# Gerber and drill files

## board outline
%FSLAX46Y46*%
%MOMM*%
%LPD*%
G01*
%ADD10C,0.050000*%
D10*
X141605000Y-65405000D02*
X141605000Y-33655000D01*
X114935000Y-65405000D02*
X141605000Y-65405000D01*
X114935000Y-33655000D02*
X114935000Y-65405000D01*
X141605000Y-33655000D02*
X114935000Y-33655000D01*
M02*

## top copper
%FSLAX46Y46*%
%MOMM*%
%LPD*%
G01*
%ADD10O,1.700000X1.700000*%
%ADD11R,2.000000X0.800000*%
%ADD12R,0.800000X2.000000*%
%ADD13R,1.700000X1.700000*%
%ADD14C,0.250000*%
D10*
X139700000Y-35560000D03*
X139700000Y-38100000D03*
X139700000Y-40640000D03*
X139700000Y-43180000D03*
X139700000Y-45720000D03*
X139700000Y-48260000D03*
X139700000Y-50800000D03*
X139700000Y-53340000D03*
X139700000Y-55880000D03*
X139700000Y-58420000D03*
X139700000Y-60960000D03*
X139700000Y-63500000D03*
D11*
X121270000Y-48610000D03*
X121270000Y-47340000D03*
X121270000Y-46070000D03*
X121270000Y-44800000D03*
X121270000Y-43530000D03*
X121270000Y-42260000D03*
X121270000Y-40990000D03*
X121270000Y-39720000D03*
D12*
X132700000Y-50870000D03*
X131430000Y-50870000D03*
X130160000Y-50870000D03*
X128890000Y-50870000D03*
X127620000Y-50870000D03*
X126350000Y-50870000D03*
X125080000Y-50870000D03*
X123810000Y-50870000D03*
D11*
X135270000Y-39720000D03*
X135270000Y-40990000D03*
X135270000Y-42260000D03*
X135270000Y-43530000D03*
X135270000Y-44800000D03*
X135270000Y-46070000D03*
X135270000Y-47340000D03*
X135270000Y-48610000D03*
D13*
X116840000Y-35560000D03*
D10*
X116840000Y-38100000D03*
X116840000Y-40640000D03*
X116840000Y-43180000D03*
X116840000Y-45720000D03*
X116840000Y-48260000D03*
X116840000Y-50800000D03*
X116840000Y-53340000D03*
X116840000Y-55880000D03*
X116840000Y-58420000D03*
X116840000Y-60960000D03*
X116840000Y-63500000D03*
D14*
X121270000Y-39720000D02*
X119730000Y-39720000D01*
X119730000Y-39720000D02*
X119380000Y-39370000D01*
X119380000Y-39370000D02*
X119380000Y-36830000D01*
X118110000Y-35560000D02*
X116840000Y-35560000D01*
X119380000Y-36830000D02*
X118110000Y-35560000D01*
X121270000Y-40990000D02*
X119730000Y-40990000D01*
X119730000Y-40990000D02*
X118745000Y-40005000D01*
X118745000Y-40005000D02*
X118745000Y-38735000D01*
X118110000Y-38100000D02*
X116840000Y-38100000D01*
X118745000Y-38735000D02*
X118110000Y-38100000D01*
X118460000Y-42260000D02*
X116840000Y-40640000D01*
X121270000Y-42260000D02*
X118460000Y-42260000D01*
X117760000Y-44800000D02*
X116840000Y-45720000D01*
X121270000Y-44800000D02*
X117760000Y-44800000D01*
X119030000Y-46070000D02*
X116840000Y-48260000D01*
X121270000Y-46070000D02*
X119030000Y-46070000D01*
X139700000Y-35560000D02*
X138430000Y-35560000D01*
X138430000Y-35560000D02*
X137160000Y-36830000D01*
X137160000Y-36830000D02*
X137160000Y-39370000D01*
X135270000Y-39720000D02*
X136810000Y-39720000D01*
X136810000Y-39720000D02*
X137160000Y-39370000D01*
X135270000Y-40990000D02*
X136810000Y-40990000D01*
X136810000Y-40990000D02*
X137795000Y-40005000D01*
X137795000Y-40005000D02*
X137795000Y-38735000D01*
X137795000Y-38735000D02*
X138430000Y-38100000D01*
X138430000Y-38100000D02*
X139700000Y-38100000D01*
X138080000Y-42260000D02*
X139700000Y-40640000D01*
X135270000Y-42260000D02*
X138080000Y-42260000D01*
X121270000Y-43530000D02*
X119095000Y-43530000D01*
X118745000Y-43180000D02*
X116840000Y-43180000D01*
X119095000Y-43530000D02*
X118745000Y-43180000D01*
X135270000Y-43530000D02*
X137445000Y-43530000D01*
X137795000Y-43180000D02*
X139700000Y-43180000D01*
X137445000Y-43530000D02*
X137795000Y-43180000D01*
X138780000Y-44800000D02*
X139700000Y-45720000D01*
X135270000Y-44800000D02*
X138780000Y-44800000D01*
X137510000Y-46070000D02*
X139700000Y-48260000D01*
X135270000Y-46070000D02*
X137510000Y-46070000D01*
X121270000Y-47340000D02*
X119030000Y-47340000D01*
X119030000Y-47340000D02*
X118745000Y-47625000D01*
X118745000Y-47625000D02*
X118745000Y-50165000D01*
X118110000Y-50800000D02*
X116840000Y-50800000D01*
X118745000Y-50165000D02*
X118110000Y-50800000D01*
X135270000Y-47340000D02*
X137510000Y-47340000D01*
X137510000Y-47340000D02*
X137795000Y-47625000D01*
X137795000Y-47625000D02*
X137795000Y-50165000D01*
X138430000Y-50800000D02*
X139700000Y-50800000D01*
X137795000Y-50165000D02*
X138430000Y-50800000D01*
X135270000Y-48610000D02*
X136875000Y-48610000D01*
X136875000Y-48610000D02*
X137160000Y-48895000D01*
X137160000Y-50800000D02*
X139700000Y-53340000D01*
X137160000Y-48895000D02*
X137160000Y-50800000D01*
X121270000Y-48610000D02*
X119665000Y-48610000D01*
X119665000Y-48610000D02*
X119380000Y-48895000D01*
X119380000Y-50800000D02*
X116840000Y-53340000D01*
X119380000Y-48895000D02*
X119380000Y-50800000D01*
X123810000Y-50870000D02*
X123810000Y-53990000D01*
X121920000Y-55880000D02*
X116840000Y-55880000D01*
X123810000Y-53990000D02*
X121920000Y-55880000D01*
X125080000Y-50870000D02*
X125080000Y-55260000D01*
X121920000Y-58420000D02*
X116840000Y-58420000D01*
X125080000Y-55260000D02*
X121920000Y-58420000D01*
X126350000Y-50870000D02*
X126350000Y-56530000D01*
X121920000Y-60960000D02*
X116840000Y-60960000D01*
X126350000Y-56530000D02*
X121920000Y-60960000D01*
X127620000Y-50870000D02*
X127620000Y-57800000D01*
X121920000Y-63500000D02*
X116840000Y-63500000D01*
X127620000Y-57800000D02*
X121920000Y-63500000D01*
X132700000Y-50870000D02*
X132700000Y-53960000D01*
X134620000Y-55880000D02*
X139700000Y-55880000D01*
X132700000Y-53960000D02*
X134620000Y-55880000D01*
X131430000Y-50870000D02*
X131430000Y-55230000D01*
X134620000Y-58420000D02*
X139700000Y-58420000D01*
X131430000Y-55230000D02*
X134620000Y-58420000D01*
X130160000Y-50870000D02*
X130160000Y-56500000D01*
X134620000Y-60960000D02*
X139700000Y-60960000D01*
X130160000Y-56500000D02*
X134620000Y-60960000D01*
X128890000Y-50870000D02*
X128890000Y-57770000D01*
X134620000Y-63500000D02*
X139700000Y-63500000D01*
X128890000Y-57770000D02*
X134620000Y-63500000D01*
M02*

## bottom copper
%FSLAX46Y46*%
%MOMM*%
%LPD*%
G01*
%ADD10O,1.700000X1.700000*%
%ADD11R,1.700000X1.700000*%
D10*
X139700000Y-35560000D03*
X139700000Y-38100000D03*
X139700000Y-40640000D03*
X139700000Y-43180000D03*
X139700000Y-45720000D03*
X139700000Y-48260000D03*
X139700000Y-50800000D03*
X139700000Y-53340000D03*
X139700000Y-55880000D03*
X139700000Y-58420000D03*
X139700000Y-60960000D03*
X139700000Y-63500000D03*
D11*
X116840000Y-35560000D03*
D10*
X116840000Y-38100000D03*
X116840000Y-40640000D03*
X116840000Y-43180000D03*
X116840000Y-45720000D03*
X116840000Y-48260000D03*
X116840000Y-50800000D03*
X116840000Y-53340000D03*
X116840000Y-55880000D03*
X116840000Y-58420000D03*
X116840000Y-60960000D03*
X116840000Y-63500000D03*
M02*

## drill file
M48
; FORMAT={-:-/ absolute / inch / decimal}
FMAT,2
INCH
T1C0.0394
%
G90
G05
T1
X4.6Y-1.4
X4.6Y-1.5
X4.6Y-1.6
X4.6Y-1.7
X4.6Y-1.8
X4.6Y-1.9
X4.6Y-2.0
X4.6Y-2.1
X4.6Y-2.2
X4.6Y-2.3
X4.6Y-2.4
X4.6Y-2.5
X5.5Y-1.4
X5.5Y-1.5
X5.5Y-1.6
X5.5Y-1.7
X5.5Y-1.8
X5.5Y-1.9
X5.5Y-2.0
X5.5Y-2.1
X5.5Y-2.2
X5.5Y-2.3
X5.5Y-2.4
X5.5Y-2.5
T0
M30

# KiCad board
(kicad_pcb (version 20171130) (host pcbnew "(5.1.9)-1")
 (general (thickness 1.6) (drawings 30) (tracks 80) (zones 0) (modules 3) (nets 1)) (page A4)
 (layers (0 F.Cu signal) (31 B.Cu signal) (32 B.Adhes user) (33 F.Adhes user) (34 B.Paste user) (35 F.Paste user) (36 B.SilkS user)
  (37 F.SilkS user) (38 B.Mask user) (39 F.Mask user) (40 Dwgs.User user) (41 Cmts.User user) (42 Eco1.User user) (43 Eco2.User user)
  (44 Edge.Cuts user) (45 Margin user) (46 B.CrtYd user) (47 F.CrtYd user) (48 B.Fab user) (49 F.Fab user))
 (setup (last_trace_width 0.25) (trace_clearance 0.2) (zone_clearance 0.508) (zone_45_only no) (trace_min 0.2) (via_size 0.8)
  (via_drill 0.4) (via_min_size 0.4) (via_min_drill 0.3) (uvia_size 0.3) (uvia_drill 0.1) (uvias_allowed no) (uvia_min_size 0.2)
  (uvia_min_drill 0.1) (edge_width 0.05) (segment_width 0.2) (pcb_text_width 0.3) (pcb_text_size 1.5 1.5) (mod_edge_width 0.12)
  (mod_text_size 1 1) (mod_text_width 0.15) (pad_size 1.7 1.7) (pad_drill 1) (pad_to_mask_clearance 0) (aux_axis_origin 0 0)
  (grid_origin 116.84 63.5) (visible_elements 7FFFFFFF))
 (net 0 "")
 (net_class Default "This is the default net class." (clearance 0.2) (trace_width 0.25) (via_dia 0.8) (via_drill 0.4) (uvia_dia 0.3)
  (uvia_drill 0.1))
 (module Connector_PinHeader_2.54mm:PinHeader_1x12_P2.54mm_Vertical (layer B.Cu) (at 139.7 63.5)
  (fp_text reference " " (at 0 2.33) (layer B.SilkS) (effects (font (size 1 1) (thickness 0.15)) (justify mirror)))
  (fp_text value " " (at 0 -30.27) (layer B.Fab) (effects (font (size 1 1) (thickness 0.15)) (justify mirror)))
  (pad 12 thru_hole oval (at 0 -27.94) (size 1.7 1.7) (drill 1) (layers *.Cu *.Mask))
  (pad 11 thru_hole oval (at 0 -25.4) (size 1.7 1.7) (drill 1) (layers *.Cu *.Mask))
  (pad 10 thru_hole oval (at 0 -22.86) (size 1.7 1.7) (drill 1) (layers *.Cu *.Mask))
  (pad 9 thru_hole oval (at 0 -20.32) (size 1.7 1.7) (drill 1) (layers *.Cu *.Mask))
  (pad 8 thru_hole oval (at 0 -17.78) (size 1.7 1.7) (drill 1) (layers *.Cu *.Mask))
  (pad 7 thru_hole oval (at 0 -15.24) (size 1.7 1.7) (drill 1) (layers *.Cu *.Mask))
  (pad 6 thru_hole oval (at 0 -12.7) (size 1.7 1.7) (drill 1) (layers *.Cu *.Mask))
  (pad 5 thru_hole oval (at 0 -10.16) (size 1.7 1.7) (drill 1) (layers *.Cu *.Mask))
  (pad 4 thru_hole oval (at 0 -7.62) (size 1.7 1.7) (drill 1) (layers *.Cu *.Mask))
  (pad 3 thru_hole oval (at 0 -5.08) (size 1.7 1.7) (drill 1) (layers *.Cu *.Mask))
  (pad 2 thru_hole oval (at 0 -2.54) (size 1.7 1.7) (drill 1) (layers *.Cu *.Mask))
  (pad 1 thru_hole oval (at 0 0) (size 1.7 1.7) (drill 1) (layers *.Cu *.Mask)))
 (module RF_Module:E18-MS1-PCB (layer F.Cu) (at 128.27 39.37)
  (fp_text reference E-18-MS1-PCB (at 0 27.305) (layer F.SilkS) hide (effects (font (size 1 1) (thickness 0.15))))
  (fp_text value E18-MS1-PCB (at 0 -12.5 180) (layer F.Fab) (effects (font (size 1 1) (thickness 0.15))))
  (pad 8 smd rect (at -7 9.24 270) (size 0.8 2) (layers F.Cu F.Paste F.Mask))
  (pad 7 smd rect (at -7 7.97 270) (size 0.8 2) (layers F.Cu F.Paste F.Mask))
  (pad 6 smd rect (at -7 6.7 270) (size 0.8 2) (layers F.Cu F.Paste F.Mask))
  (pad 5 smd rect (at -7 5.43 270) (size 0.8 2) (layers F.Cu F.Paste F.Mask))
  (pad 4 smd rect (at -7 4.16 270) (size 0.8 2) (layers F.Cu F.Paste F.Mask))
  (pad 3 smd rect (at -7 2.89 270) (size 0.8 2) (layers F.Cu F.Paste F.Mask))
  (pad 2 smd rect (at -7 1.62 270) (size 0.8 2) (layers F.Cu F.Paste F.Mask))
  (pad 1 smd rect (at -7 0.35 270) (size 0.8 2) (layers F.Cu F.Paste F.Mask))
  (pad 16 smd rect (at 4.43 11.5 180) (size 0.8 2) (layers F.Cu F.Paste F.Mask))
  (pad 15 smd rect (at 3.16 11.5 180) (size 0.8 2) (layers F.Cu F.Paste F.Mask))
  (pad 14 smd rect (at 1.89 11.5 180) (size 0.8 2) (layers F.Cu F.Paste F.Mask))
  (pad 13 smd rect (at 0.62 11.5 180) (size 0.8 2) (layers F.Cu F.Paste F.Mask))
  (pad 12 smd rect (at -0.65 11.5 180) (size 0.8 2) (layers F.Cu F.Paste F.Mask))
  (pad 11 smd rect (at -1.92 11.5 180) (size 0.8 2) (layers F.Cu F.Paste F.Mask))
  (pad 10 smd rect (at -3.19 11.5 180) (size 0.8 2) (layers F.Cu F.Paste F.Mask))
  (pad 9 smd rect (at -4.46 11.5 180) (size 0.8 2) (layers F.Cu F.Paste F.Mask))
  (pad 24 smd rect (at 7 0.35 90) (size 0.8 2) (layers F.Cu F.Paste F.Mask))
  (pad 23 smd rect (at 7 1.62 90) (size 0.8 2) (layers F.Cu F.Paste F.Mask))
  (pad 22 smd rect (at 7 2.89 90) (size 0.8 2) (layers F.Cu F.Paste F.Mask))
  (pad 21 smd rect (at 7 4.16 90) (size 0.8 2) (layers F.Cu F.Paste F.Mask))
  (pad 20 smd rect (at 7 5.43 90) (size 0.8 2) (layers F.Cu F.Paste F.Mask))
  (pad 19 smd rect (at 7 6.7 90) (size 0.8 2) (layers F.Cu F.Paste F.Mask))
  (pad 18 smd rect (at 7 7.97 90) (size 0.8 2) (layers F.Cu F.Paste F.Mask))
  (pad 17 smd rect (at 7 9.24 90) (size 0.8 2) (layers F.Cu F.Paste F.Mask)))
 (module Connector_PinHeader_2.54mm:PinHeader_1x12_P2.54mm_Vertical (layer B.Cu) (at 116.84 63.5)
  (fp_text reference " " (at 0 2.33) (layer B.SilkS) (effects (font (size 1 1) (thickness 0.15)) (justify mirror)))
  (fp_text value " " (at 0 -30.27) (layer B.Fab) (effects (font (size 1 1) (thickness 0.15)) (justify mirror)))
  (pad 12 thru_hole rect (at 0 -27.94) (size 1.7 1.7) (drill 1) (layers *.Cu *.Mask))
  (pad 11 thru_hole oval (at 0 -25.4) (size 1.7 1.7) (drill 1) (layers *.Cu *.Mask))
  (pad 10 thru_hole oval (at 0 -22.86) (size 1.7 1.7) (drill 1) (layers *.Cu *.Mask))
  (pad 9 thru_hole oval (at 0 -20.32) (size 1.7 1.7) (drill 1) (layers *.Cu *.Mask))
  (pad 8 thru_hole oval (at 0 -17.78) (size 1.7 1.7) (drill 1) (layers *.Cu *.Mask))
  (pad 7 thru_hole oval (at 0 -15.24) (size 1.7 1.7) (drill 1) (layers *.Cu *.Mask))
  (pad 6 thru_hole oval (at 0 -12.7) (size 1.7 1.7) (drill 1) (layers *.Cu *.Mask))
  (pad 5 thru_hole oval (at 0 -10.16) (size 1.7 1.7) (drill 1) (layers *.Cu *.Mask))
  (pad 4 thru_hole oval (at 0 -7.62) (size 1.7 1.7) (drill 1) (layers *.Cu *.Mask))
  (pad 3 thru_hole oval (at 0 -5.08) (size 1.7 1.7) (drill 1) (layers *.Cu *.Mask))
  (pad 2 thru_hole oval (at 0 -2.54) (size 1.7 1.7) (drill 1) (layers *.Cu *.Mask))
  (pad 1 thru_hole oval (at 0 0) (size 1.7 1.7) (drill 1) (layers *.Cu *.Mask)))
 (gr_line (start 141.605 65.405) (end 141.605 33.655) (layer Edge.Cuts) (width 0.05))
 (gr_line (start 114.935 65.405) (end 141.605 65.405) (layer Edge.Cuts) (width 0.05))
 (gr_line (start 114.935 33.655) (end 114.935 65.405) (layer Edge.Cuts) (width 0.05))
 (gr_line (start 141.605 33.655) (end 114.935 33.655) (layer Edge.Cuts) (width 0.05))
 (segment (start 121.27 39.72) (end 119.73 39.72) (width 0.25) (layer F.Cu) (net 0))
 (segment (start 119.73 39.72) (end 119.38 39.37) (width 0.25) (layer F.Cu) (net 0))
 (segment (start 119.38 39.37) (end 119.38 36.83) (width 0.25) (layer F.Cu) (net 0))
 (segment (start 118.11 35.56) (end 116.84 35.56) (width 0.25) (layer F.Cu) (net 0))
 (segment (start 119.38 36.83) (end 118.11 35.56) (width 0.25) (layer F.Cu) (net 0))
 (segment (start 121.27 40.99) (end 119.73 40.99) (width 0.25) (layer F.Cu) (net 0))
 (segment (start 119.73 40.99) (end 118.745 40.005) (width 0.25) (layer F.Cu) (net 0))
 (segment (start 118.745 40.005) (end 118.745 38.735) (width 0.25) (layer F.Cu) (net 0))
 (segment (start 118.11 38.1) (end 116.84 38.1) (width 0.25) (layer F.Cu) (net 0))
 (segment (start 118.745 38.735) (end 118.11 38.1) (width 0.25) (layer F.Cu) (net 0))
 (segment (start 118.46 42.26) (end 116.84 40.64) (width 0.25) (layer F.Cu) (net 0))
 (segment (start 121.27 42.26) (end 118.46 42.26) (width 0.25) (layer F.Cu) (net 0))
 (segment (start 117.76 44.8) (end 116.84 45.72) (width 0.25) (layer F.Cu) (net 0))
 (segment (start 121.27 44.8) (end 117.76 44.8) (width 0.25) (layer F.Cu) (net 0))
 (segment (start 119.03 46.07) (end 116.84 48.26) (width 0.25) (layer F.Cu) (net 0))
 (segment (start 121.27 46.07) (end 119.03 46.07) (width 0.25) (layer F.Cu) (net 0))
 (segment (start 139.7 35.56) (end 138.43 35.56) (width 0.25) (layer F.Cu) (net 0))
 (segment (start 138.43 35.56) (end 137.16 36.83) (width 0.25) (layer F.Cu) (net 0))
 (segment (start 137.16 36.83) (end 137.16 39.37) (width 0.25) (layer F.Cu) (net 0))
 (segment (start 135.27 39.72) (end 136.81 39.72) (width 0.25) (layer F.Cu) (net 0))
 (segment (start 136.81 39.72) (end 137.16 39.37) (width 0.25) (layer F.Cu) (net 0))
 (segment (start 135.27 40.99) (end 136.81 40.99) (width 0.25) (layer F.Cu) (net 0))
 (segment (start 136.81 40.99) (end 137.795 40.005) (width 0.25) (layer F.Cu) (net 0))
 (segment (start 137.795 40.005) (end 137.795 38.735) (width 0.25) (layer F.Cu) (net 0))
 (segment (start 137.795 38.735) (end 138.43 38.1) (width 0.25) (layer F.Cu) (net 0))
 (segment (start 138.43 38.1) (end 139.7 38.1) (width 0.25) (layer F.Cu) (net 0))
 (segment (start 138.08 42.26) (end 139.7 40.64) (width 0.25) (layer F.Cu) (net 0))
 (segment (start 135.27 42.26) (end 138.08 42.26) (width 0.25) (layer F.Cu) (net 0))
 (segment (start 121.27 43.53) (end 119.095 43.53) (width 0.25) (layer F.Cu) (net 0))
 (segment (start 118.745 43.18) (end 116.84 43.18) (width 0.25) (layer F.Cu) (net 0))
 (segment (start 119.095 43.53) (end 118.745 43.18) (width 0.25) (layer F.Cu) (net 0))
 (segment (start 135.27 43.53) (end 137.445 43.53) (width 0.25) (layer F.Cu) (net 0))
 (segment (start 137.795 43.18) (end 139.7 43.18) (width 0.25) (layer F.Cu) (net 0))
 (segment (start 137.445 43.53) (end 137.795 43.18) (width 0.25) (layer F.Cu) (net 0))
 (segment (start 138.78 44.8) (end 139.7 45.72) (width 0.25) (layer F.Cu) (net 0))
 (segment (start 135.27 44.8) (end 138.78 44.8) (width 0.25) (layer F.Cu) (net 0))
 (segment (start 137.51 46.07) (end 139.7 48.26) (width 0.25) (layer F.Cu) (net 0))
 (segment (start 135.27 46.07) (end 137.51 46.07) (width 0.25) (layer F.Cu) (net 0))
 (segment (start 121.27 47.34) (end 119.03 47.34) (width 0.25) (layer F.Cu) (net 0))
 (segment (start 119.03 47.34) (end 118.745 47.625) (width 0.25) (layer F.Cu) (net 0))
 (segment (start 118.745 47.625) (end 118.745 50.165) (width 0.25) (layer F.Cu) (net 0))
 (segment (start 118.11 50.8) (end 116.84 50.8) (width 0.25) (layer F.Cu) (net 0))
 (segment (start 118.745 50.165) (end 118.11 50.8) (width 0.25) (layer F.Cu) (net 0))
 (segment (start 135.27 47.34) (end 137.51 47.34) (width 0.25) (layer F.Cu) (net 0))
 (segment (start 137.51 47.34) (end 137.795 47.625) (width 0.25) (layer F.Cu) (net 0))
 (segment (start 137.795 47.625) (end 137.795 50.165) (width 0.25) (layer F.Cu) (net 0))
 (segment (start 138.43 50.8) (end 139.7 50.8) (width 0.25) (layer F.Cu) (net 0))
 (segment (start 137.795 50.165) (end 138.43 50.8) (width 0.25) (layer F.Cu) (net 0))
 (segment (start 135.27 48.61) (end 136.875 48.61) (width 0.25) (layer F.Cu) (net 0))
 (segment (start 136.875 48.61) (end 137.16 48.895) (width 0.25) (layer F.Cu) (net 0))
 (segment (start 137.16 50.8) (end 139.7 53.34) (width 0.25) (layer F.Cu) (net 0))
 (segment (start 137.16 48.895) (end 137.16 50.8) (width 0.25) (layer F.Cu) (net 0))
 (segment (start 121.27 48.61) (end 119.665 48.61) (width 0.25) (layer F.Cu) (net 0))
 (segment (start 119.665 48.61) (end 119.38 48.895) (width 0.25) (layer F.Cu) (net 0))
 (segment (start 119.38 50.8) (end 116.84 53.34) (width 0.25) (layer F.Cu) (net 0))
 (segment (start 119.38 48.895) (end 119.38 50.8) (width 0.25) (layer F.Cu) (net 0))
 (segment (start 123.81 50.87) (end 123.81 53.99) (width 0.25) (layer F.Cu) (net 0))
 (segment (start 121.92 55.88) (end 116.84 55.88) (width 0.25) (layer F.Cu) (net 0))
 (segment (start 123.81 53.99) (end 121.92 55.88) (width 0.25) (layer F.Cu) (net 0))
 (segment (start 125.08 50.87) (end 125.08 55.26) (width 0.25) (layer F.Cu) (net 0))
 (segment (start 121.92 58.42) (end 116.84 58.42) (width 0.25) (layer F.Cu) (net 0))
 (segment (start 125.08 55.26) (end 121.92 58.42) (width 0.25) (layer F.Cu) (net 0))
 (segment (start 126.35 50.87) (end 126.35 56.53) (width 0.25) (layer F.Cu) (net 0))
 (segment (start 121.92 60.96) (end 116.84 60.96) (width 0.25) (layer F.Cu) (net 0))
 (segment (start 126.35 56.53) (end 121.92 60.96) (width 0.25) (layer F.Cu) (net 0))
 (segment (start 127.62 50.87) (end 127.62 57.8) (width 0.25) (layer F.Cu) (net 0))
 (segment (start 121.92 63.5) (end 116.84 63.5) (width 0.25) (layer F.Cu) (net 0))
 (segment (start 127.62 57.8) (end 121.92 63.5) (width 0.25) (layer F.Cu) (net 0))
 (segment (start 132.7 50.87) (end 132.7 53.96) (width 0.25) (layer F.Cu) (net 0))
 (segment (start 134.62 55.88) (end 139.7 55.88) (width 0.25) (layer F.Cu) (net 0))
 (segment (start 132.7 53.96) (end 134.62 55.88) (width 0.25) (layer F.Cu) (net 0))
 (segment (start 131.43 50.87) (end 131.43 55.23) (width 0.25) (layer F.Cu) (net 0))
 (segment (start 134.62 58.42) (end 139.7 58.42) (width 0.25) (layer F.Cu) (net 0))
 (segment (start 131.43 55.23) (end 134.62 58.42) (width 0.25) (layer F.Cu) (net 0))
 (segment (start 130.16 50.87) (end 130.16 56.5) (width 0.25) (layer F.Cu) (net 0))
 (segment (start 134.62 60.96) (end 139.7 60.96) (width 0.25) (layer F.Cu) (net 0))
 (segment (start 130.16 56.5) (end 134.62 60.96) (width 0.25) (layer F.Cu) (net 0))
 (segment (start 128.89 50.87) (end 128.89 57.77) (width 0.25) (layer F.Cu) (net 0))
 (segment (start 134.62 63.5) (end 139.7 63.5) (width 0.25) (layer F.Cu) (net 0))
 (segment (start 128.89 57.77) (end 134.62 63.5) (width 0.25) (layer F.Cu) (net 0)))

